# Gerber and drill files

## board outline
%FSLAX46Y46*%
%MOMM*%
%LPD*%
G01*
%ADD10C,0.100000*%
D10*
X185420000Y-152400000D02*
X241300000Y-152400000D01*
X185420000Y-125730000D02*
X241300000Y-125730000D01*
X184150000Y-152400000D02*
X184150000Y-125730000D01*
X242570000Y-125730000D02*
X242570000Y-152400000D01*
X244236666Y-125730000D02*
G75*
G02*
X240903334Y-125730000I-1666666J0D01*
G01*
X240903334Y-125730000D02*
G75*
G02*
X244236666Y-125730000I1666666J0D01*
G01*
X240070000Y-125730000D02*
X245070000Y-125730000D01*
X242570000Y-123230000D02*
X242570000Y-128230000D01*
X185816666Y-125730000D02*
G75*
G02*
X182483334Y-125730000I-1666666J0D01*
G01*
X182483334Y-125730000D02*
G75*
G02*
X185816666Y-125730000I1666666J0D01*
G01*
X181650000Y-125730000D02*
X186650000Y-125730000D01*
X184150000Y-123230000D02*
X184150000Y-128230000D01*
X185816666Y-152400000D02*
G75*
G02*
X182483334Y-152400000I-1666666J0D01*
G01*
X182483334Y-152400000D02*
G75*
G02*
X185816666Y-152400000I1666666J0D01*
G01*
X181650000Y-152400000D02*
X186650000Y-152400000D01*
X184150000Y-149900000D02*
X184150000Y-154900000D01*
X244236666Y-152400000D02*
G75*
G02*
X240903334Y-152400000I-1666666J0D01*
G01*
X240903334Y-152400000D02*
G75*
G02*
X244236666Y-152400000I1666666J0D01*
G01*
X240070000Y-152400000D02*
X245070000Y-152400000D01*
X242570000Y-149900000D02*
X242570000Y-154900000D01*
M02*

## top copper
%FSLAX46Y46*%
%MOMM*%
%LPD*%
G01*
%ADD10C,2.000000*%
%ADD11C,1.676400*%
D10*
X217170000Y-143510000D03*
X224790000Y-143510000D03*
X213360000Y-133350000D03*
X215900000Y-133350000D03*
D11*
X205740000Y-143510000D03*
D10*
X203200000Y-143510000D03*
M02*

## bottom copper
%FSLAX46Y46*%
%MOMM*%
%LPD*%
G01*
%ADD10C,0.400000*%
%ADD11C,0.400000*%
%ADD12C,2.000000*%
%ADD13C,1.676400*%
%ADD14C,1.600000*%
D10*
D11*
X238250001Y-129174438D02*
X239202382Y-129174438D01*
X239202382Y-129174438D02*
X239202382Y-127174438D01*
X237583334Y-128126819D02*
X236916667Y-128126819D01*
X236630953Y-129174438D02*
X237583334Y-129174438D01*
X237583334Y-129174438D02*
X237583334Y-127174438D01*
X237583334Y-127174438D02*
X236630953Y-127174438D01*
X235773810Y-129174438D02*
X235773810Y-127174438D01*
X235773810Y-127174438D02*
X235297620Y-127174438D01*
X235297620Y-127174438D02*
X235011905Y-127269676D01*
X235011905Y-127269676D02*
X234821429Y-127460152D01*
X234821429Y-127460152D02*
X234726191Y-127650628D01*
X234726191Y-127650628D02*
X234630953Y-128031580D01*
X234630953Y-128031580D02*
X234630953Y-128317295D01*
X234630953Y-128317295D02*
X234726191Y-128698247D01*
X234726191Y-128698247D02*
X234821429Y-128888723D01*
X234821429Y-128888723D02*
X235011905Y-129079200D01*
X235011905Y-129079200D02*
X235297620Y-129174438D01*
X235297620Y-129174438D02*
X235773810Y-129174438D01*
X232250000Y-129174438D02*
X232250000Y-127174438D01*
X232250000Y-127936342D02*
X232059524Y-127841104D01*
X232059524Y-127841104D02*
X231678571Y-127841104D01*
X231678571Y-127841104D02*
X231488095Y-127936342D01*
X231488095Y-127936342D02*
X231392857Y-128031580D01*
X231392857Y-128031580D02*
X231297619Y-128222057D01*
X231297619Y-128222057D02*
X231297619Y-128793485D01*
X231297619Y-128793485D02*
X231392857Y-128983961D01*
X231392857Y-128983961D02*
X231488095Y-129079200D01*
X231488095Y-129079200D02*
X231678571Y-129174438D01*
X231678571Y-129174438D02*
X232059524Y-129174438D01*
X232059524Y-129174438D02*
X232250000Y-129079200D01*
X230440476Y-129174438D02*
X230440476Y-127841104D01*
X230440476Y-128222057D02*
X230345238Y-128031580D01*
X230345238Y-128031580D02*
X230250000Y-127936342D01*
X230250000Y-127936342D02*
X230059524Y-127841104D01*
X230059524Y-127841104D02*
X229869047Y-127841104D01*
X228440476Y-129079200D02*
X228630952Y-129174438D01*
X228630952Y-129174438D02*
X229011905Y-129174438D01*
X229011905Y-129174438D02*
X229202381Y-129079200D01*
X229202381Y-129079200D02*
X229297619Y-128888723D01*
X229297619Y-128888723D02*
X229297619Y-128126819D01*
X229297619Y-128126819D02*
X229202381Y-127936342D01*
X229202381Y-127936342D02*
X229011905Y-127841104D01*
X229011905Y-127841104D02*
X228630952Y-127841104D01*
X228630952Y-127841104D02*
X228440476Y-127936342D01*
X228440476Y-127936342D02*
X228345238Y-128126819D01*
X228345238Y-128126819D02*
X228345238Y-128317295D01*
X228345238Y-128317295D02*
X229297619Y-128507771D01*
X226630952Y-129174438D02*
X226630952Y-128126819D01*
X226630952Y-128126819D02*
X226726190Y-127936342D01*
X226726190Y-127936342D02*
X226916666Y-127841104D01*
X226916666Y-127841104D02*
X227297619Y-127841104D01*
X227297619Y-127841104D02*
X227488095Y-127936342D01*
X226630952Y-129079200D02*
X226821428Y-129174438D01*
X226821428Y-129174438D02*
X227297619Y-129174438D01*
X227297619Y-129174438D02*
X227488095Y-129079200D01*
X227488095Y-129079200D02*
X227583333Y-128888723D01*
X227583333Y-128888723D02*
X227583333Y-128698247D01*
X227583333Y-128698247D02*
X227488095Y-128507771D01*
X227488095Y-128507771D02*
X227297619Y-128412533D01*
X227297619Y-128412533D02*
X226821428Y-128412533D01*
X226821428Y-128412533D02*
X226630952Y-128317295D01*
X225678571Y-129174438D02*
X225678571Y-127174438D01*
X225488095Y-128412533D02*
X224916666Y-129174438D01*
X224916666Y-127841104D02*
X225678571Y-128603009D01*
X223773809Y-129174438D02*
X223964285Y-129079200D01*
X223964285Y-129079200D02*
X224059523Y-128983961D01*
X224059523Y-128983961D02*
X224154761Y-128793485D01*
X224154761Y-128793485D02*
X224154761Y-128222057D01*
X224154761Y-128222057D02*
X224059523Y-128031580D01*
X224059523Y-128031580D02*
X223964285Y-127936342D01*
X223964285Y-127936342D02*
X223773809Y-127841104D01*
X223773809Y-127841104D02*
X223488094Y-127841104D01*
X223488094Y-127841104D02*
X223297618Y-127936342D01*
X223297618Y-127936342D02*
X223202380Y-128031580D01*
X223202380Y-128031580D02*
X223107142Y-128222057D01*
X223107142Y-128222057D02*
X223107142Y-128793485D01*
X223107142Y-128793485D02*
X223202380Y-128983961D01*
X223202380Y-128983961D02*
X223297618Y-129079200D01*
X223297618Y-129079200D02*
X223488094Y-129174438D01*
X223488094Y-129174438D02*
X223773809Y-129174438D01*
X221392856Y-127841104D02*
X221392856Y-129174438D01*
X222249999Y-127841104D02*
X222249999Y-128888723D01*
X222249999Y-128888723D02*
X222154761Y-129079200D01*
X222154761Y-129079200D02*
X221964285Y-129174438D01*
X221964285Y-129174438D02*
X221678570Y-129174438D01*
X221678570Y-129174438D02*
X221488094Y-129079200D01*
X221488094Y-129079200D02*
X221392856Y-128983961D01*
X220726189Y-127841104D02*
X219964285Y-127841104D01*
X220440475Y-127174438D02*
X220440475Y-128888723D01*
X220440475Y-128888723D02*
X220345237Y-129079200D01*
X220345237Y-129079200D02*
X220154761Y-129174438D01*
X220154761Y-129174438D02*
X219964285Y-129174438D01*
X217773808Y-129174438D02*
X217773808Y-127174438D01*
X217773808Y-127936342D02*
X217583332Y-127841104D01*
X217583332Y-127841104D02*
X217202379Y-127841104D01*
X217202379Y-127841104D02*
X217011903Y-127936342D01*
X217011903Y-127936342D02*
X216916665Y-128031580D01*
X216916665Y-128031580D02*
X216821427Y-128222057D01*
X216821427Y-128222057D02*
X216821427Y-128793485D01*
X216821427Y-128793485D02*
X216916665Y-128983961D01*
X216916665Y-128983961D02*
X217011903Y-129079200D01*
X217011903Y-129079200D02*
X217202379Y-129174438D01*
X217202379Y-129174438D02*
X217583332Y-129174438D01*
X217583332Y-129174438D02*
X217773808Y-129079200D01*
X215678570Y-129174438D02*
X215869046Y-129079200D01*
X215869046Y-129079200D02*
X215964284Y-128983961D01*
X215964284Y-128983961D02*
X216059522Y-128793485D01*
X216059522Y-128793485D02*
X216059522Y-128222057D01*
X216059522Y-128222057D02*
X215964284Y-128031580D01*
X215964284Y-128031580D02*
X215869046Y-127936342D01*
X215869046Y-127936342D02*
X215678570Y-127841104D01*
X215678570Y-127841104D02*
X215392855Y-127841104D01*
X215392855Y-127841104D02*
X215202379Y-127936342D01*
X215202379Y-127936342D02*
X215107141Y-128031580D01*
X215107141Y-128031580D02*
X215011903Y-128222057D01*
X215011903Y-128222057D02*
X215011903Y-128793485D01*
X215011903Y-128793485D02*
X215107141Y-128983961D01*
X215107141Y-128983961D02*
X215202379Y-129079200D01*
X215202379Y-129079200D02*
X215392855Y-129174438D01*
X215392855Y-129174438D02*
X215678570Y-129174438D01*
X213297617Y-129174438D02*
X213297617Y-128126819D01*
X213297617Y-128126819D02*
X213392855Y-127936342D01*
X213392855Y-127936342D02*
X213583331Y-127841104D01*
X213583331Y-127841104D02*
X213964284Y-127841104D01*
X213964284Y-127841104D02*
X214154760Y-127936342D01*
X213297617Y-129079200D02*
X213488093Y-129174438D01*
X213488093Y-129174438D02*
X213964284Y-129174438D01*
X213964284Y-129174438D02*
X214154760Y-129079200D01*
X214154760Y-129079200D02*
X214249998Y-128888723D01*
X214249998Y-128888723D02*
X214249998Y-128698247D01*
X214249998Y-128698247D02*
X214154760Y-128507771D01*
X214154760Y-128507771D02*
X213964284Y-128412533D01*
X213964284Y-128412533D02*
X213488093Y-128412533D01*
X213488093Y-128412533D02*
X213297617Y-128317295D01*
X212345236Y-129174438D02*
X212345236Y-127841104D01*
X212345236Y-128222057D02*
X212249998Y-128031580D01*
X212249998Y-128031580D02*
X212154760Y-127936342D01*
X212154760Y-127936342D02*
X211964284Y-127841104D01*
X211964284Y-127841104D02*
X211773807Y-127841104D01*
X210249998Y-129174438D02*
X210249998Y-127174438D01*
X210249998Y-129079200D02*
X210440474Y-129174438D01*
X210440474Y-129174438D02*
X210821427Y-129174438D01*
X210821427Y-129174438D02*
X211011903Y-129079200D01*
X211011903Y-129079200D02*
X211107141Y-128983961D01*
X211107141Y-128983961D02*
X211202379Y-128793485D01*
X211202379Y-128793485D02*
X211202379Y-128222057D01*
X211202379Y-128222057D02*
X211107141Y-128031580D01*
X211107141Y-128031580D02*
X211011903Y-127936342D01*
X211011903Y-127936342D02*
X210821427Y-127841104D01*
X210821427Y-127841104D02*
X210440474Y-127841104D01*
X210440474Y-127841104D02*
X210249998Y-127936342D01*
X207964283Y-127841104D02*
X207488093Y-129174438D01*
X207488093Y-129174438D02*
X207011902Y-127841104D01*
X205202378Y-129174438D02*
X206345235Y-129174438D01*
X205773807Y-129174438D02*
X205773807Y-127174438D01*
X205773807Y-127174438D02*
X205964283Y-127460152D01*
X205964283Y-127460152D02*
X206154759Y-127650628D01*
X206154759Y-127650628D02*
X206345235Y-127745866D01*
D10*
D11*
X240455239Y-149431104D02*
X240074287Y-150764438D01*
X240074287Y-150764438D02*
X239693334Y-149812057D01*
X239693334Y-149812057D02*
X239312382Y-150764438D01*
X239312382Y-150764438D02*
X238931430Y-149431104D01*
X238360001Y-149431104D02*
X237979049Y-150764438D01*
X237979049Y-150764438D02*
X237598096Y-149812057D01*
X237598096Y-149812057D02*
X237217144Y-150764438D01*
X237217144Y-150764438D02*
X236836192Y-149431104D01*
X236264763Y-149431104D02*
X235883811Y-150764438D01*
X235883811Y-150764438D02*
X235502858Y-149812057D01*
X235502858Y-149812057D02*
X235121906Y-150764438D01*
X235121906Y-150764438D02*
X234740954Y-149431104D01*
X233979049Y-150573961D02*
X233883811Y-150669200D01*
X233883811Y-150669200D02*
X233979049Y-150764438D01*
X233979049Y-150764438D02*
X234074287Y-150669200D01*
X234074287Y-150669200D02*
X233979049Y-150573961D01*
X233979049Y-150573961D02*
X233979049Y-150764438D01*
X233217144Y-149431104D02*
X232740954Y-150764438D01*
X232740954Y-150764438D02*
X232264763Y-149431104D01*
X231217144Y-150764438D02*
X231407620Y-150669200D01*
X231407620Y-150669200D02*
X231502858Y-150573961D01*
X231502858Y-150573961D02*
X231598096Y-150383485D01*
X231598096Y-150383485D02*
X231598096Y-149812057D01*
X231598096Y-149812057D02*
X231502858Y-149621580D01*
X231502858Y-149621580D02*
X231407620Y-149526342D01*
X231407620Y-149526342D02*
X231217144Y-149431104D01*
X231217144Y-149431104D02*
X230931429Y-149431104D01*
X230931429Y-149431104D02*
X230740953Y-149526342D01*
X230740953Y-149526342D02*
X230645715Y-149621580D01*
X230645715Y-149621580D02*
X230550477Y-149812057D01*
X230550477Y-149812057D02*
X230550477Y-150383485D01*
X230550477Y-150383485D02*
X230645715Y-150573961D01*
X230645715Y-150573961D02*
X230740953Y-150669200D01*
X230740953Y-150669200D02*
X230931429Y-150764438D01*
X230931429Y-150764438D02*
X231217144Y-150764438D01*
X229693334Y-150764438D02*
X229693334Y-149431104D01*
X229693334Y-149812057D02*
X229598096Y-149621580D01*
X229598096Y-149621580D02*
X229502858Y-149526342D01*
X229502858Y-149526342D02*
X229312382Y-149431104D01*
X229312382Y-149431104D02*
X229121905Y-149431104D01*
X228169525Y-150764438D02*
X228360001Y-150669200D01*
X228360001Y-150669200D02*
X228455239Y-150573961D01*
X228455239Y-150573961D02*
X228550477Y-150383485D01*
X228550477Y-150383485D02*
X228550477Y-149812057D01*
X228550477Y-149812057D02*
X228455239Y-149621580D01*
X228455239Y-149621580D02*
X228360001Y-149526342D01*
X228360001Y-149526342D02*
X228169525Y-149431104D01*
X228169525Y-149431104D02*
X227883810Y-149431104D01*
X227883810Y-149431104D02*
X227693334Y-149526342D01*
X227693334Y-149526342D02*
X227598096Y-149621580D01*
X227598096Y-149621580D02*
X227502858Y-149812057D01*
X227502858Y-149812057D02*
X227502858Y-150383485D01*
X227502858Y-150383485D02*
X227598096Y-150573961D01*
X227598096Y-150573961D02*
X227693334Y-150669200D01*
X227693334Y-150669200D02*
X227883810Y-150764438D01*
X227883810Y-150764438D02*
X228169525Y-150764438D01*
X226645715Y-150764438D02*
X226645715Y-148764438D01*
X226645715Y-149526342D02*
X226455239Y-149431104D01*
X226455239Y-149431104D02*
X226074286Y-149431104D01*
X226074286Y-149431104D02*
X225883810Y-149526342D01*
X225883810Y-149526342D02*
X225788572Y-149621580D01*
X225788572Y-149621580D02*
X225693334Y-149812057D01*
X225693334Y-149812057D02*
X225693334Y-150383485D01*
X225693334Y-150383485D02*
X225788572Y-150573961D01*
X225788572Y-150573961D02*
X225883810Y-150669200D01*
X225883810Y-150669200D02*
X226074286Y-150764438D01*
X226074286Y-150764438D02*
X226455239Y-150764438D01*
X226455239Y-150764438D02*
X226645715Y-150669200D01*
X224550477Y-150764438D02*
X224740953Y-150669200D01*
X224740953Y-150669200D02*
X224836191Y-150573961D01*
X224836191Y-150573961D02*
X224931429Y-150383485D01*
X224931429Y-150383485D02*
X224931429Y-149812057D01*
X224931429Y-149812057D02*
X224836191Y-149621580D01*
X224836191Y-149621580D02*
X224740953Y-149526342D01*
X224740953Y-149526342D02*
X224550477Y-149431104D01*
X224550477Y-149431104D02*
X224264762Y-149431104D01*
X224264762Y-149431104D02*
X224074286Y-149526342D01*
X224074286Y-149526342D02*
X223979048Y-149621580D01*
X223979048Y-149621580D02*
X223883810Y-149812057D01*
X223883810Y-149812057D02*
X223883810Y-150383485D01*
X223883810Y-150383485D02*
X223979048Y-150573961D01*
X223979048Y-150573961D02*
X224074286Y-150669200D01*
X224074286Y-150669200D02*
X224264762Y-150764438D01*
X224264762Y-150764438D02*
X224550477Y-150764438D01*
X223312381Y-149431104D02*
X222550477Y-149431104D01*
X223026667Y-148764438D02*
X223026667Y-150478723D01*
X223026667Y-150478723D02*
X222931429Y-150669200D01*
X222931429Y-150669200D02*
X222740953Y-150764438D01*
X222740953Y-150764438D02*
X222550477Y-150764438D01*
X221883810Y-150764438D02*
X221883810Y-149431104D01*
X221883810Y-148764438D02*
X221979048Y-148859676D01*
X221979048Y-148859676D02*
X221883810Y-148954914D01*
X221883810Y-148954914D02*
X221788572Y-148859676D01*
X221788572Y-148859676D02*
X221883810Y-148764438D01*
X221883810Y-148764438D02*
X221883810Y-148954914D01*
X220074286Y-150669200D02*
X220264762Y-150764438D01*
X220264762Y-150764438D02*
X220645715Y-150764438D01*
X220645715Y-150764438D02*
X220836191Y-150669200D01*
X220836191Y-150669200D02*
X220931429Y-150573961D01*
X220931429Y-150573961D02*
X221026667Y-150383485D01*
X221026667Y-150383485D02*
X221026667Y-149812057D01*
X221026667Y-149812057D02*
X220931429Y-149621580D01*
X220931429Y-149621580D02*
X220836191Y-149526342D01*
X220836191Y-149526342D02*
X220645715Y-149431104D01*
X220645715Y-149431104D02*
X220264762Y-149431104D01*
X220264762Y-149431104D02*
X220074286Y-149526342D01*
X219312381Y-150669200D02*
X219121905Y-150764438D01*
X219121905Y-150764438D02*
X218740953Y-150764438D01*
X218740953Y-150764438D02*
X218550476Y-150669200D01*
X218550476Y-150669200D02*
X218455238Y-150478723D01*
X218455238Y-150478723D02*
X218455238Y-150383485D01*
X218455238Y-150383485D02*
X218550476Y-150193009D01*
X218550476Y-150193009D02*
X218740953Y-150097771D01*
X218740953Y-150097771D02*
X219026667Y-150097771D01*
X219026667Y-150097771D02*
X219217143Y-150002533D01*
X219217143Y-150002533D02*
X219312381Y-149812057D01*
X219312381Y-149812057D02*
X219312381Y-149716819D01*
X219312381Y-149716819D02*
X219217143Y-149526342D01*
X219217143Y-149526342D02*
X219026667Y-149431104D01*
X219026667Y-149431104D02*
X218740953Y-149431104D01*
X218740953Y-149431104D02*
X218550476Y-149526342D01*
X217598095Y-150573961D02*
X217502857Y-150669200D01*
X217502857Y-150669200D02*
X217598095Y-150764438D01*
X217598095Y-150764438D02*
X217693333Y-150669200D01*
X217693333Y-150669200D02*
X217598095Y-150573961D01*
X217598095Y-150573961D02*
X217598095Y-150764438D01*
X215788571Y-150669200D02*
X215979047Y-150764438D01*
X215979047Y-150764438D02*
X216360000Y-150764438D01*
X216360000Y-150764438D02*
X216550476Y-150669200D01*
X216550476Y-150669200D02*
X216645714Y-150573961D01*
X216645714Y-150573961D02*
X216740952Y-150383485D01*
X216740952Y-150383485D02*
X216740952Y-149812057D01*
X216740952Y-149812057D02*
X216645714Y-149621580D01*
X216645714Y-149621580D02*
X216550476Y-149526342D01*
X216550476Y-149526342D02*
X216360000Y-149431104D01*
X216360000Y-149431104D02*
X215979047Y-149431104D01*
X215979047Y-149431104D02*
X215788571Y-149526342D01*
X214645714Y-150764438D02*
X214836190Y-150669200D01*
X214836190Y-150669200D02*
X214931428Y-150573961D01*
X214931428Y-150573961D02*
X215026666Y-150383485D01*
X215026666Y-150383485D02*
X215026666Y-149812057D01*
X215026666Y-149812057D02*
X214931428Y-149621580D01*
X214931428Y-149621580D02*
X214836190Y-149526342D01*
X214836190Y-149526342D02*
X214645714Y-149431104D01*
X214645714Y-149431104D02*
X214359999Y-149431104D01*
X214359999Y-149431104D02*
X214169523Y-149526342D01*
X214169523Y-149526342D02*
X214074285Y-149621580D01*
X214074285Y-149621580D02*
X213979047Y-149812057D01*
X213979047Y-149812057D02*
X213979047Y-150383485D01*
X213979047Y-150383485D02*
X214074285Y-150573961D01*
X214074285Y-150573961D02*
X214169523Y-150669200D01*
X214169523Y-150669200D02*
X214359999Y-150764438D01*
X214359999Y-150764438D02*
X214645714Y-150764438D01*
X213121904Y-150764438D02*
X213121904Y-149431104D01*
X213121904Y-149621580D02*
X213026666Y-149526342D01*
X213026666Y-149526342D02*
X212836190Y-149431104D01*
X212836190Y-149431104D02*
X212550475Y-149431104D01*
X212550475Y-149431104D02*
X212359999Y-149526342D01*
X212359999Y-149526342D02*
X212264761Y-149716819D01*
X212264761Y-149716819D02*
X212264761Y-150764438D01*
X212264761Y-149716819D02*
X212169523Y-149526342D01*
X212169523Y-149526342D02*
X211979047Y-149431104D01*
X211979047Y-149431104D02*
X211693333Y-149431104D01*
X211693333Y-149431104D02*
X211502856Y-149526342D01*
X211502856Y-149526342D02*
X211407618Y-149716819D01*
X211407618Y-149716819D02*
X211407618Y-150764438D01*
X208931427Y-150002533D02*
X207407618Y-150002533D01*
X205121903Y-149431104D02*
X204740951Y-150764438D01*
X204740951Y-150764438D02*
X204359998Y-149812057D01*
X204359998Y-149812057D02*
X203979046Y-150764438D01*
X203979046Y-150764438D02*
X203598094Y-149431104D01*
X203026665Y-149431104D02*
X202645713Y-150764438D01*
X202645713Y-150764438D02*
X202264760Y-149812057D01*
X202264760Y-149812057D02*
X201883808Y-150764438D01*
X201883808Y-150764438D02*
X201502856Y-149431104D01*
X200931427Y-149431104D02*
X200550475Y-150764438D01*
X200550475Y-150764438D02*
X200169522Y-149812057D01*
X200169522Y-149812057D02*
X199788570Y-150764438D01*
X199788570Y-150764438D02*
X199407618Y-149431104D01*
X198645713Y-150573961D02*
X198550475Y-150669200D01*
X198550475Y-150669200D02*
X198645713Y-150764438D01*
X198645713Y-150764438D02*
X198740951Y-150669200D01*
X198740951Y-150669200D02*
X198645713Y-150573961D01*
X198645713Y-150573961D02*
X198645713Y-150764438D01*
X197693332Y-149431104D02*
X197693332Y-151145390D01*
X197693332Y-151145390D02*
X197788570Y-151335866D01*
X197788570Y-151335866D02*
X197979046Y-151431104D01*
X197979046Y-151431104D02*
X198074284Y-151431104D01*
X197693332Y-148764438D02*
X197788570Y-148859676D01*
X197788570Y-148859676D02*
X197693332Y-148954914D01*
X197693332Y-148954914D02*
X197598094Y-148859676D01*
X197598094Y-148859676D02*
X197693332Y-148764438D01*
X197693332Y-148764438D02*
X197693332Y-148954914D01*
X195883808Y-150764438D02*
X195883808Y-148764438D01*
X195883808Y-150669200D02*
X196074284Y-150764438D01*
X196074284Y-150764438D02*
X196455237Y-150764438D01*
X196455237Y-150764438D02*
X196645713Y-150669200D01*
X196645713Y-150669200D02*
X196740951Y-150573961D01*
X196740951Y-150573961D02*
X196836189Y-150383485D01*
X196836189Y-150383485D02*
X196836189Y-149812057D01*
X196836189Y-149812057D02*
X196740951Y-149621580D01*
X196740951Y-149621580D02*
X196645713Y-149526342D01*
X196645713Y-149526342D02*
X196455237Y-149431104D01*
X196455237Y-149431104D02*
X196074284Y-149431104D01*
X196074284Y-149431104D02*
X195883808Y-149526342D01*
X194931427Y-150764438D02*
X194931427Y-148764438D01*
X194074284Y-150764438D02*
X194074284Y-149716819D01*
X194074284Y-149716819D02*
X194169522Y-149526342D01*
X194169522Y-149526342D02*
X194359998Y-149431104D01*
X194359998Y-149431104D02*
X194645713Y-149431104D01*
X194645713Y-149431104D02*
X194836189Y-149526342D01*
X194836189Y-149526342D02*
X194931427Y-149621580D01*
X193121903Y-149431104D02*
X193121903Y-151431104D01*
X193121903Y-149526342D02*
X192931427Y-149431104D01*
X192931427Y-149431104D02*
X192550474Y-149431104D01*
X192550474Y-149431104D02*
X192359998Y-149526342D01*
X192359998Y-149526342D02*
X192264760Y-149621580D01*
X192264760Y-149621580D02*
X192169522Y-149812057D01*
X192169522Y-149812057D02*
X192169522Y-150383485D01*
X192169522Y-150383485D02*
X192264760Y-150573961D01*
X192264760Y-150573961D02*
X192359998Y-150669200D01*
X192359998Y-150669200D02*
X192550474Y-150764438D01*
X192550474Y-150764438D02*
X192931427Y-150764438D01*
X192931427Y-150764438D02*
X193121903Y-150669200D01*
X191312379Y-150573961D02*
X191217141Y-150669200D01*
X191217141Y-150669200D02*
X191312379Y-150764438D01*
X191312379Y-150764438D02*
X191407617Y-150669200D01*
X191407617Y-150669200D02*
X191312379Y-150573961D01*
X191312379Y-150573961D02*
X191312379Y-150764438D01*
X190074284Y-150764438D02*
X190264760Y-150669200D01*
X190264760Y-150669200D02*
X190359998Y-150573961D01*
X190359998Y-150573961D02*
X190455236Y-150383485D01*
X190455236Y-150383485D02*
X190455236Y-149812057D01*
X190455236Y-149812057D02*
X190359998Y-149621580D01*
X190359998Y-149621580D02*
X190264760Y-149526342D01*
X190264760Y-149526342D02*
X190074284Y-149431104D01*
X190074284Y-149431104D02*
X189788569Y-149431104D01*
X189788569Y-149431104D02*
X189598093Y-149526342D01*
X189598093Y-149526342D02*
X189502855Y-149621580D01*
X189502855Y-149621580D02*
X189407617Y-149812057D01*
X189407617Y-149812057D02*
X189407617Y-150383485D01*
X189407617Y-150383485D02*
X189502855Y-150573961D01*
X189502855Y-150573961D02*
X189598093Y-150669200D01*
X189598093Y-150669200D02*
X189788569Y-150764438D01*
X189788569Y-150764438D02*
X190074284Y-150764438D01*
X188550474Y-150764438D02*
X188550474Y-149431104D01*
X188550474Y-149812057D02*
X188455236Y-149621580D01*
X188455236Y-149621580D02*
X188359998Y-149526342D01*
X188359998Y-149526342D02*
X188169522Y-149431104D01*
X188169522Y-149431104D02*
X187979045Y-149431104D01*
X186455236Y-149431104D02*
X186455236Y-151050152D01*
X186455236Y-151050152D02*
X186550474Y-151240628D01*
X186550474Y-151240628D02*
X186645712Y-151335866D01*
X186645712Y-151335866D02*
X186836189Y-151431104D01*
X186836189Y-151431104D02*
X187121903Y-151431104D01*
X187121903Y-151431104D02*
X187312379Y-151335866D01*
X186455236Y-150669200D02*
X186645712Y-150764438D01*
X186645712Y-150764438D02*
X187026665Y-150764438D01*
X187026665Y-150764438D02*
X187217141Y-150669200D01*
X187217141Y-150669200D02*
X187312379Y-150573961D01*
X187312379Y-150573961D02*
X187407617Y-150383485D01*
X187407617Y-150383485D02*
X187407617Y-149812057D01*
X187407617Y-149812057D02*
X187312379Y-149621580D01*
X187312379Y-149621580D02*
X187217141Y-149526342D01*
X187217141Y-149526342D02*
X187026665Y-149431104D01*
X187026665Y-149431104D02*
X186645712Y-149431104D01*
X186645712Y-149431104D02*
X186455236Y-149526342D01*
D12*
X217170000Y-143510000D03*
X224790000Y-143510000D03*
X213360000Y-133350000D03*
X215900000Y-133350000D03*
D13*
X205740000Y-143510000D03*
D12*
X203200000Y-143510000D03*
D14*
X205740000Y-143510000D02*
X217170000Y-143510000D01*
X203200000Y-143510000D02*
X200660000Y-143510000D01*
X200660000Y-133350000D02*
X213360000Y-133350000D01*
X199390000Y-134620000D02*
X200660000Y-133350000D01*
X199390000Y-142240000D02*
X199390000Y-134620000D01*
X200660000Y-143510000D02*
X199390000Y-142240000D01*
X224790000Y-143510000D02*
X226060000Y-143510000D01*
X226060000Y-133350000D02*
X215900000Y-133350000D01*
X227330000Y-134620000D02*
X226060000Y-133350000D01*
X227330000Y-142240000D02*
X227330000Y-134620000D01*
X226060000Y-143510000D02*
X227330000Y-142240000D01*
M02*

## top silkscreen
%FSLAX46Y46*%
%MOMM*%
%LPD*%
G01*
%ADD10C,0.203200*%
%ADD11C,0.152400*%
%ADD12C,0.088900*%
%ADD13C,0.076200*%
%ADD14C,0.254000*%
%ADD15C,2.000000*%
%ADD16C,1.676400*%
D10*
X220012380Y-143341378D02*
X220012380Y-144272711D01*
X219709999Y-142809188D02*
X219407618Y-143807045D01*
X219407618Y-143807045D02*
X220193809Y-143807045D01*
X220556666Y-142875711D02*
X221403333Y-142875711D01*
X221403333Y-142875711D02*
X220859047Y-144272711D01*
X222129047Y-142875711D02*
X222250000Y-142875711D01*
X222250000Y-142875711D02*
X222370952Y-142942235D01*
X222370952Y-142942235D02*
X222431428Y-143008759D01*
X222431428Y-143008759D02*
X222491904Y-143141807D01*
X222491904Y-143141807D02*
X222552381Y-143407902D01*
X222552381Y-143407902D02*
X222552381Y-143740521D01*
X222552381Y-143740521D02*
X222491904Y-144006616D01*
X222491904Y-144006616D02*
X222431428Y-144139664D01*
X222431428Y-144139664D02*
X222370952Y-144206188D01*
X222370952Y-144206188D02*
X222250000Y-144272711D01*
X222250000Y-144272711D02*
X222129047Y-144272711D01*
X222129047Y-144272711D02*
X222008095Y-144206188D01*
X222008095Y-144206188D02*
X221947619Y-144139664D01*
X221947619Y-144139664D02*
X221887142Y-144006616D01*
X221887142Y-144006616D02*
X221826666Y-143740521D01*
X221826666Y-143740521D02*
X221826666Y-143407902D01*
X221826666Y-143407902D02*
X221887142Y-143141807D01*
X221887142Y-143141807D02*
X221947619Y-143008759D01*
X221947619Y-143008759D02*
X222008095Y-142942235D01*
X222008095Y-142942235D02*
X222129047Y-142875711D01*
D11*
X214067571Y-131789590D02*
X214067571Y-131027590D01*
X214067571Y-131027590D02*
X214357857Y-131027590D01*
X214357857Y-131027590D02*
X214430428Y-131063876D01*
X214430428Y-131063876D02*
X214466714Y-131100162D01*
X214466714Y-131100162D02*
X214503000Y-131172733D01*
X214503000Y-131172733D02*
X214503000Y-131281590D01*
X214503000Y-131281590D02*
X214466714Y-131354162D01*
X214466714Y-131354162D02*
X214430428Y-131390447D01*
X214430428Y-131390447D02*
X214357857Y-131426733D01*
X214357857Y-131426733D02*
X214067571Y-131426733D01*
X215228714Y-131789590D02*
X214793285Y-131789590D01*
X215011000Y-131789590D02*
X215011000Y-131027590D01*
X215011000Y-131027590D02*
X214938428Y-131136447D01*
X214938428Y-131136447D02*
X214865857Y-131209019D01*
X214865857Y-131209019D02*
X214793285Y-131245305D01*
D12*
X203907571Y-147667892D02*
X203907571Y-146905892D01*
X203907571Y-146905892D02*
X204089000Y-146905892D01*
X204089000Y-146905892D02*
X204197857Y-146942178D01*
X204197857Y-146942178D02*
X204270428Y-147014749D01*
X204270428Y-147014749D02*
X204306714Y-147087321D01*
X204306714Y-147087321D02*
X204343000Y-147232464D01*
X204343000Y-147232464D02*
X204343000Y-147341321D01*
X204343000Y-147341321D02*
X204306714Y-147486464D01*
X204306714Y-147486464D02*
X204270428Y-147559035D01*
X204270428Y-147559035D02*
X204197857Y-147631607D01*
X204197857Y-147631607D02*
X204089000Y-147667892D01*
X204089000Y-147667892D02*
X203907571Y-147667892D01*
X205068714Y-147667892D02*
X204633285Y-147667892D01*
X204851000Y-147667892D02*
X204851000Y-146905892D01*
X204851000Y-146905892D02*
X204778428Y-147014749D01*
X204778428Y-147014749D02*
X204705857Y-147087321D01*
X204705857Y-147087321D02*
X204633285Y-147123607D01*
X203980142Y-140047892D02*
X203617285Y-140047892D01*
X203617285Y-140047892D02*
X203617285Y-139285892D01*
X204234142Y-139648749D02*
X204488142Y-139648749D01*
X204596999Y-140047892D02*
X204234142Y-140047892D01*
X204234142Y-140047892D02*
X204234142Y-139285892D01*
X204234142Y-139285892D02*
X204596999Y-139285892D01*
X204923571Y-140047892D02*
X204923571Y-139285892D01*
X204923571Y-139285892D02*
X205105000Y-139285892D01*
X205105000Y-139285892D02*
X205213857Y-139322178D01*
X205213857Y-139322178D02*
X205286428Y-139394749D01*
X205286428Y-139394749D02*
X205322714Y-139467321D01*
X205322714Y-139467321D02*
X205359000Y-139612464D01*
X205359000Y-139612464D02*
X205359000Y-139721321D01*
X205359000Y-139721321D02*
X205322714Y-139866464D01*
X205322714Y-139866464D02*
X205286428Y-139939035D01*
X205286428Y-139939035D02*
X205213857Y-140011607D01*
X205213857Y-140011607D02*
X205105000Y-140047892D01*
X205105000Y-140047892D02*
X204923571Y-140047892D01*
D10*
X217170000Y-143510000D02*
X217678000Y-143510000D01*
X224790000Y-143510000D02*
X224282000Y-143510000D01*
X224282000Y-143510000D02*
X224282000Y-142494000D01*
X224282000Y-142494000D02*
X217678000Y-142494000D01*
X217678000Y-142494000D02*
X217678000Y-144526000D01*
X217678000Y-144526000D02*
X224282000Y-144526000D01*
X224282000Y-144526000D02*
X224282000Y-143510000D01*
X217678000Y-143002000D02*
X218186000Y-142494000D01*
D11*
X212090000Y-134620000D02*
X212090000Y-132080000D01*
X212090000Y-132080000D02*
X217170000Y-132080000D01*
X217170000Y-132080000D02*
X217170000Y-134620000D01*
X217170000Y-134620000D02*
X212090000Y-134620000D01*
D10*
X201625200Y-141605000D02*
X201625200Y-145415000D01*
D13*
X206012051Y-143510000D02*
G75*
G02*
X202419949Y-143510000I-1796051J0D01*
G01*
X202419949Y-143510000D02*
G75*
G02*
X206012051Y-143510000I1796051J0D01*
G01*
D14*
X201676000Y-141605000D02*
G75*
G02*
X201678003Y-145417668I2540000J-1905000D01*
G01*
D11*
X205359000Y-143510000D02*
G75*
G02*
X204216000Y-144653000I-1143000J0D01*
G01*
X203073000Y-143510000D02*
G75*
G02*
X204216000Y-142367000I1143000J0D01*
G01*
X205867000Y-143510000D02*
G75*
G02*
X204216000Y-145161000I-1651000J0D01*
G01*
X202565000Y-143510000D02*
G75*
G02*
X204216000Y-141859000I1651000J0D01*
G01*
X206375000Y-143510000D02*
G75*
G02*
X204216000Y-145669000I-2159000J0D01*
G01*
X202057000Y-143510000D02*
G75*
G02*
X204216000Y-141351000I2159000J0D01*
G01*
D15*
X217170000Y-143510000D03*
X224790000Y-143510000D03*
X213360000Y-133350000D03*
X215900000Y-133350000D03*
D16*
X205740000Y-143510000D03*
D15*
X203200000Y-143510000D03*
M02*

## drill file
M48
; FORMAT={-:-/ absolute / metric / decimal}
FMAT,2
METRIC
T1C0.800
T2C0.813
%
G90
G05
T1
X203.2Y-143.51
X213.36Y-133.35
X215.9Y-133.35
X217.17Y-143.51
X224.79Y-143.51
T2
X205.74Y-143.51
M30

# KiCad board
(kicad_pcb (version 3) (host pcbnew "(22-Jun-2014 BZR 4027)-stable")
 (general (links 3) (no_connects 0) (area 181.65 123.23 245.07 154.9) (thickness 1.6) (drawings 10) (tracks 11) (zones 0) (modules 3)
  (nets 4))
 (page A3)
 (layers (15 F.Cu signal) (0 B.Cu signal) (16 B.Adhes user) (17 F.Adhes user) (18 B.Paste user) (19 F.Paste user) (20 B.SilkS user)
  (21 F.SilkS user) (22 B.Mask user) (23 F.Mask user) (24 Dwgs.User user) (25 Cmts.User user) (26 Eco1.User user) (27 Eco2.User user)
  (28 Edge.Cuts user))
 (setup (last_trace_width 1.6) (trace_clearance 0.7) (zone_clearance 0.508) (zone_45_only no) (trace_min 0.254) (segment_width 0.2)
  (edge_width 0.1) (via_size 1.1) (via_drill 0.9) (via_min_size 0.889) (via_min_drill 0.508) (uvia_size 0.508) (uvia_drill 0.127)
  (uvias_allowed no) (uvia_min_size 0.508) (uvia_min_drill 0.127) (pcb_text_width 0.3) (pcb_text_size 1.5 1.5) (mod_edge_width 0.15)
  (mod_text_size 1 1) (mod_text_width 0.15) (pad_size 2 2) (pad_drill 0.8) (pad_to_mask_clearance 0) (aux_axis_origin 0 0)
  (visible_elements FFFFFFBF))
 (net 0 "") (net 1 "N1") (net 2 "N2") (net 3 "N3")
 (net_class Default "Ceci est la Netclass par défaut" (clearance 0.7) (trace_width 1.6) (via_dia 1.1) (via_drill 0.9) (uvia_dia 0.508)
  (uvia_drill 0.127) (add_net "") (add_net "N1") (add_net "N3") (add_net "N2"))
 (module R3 (layer F.Cu) (at 220.98 143.51) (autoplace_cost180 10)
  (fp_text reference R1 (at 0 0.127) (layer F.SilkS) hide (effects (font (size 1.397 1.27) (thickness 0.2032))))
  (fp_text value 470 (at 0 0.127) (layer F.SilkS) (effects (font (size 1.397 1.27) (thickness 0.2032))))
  (fp_line (start -3.81 0) (end -3.302 0) (layer F.SilkS) (width 0.2032))
  (fp_line (start 3.81 0) (end 3.302 0) (layer F.SilkS) (width 0.2032))
  (fp_line (start 3.302 0) (end 3.302 -1.016) (layer F.SilkS) (width 0.2032))
  (fp_line (start 3.302 -1.016) (end -3.302 -1.016) (layer F.SilkS) (width 0.2032))
  (fp_line (start -3.302 -1.016) (end -3.302 1.016) (layer F.SilkS) (width 0.2032))
  (fp_line (start -3.302 1.016) (end 3.302 1.016) (layer F.SilkS) (width 0.2032))
  (fp_line (start 3.302 1.016) (end 3.302 0) (layer F.SilkS) (width 0.2032))
  (fp_line (start -3.302 -0.508) (end -2.794 -1.016) (layer F.SilkS) (width 0.2032))
  (pad 1 thru_hole circle (at -3.81 0) (size 2 2) (drill 0.8) (layers *.Cu *.Mask F.SilkS) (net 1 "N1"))
  (pad 2 thru_hole circle (at 3.81 0) (size 2 2) (drill 0.8) (layers *.Cu *.Mask F.SilkS) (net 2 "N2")))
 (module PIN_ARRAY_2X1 (layer F.Cu) (at 214.63 133.35)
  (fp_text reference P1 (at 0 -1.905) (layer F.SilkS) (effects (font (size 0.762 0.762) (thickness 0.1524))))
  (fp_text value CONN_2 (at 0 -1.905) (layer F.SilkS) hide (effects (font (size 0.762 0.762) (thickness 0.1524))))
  (fp_line (start -2.54 1.27) (end -2.54 -1.27) (layer F.SilkS) (width 0.1524))
  (fp_line (start -2.54 -1.27) (end 2.54 -1.27) (layer F.SilkS) (width 0.1524))
  (fp_line (start 2.54 -1.27) (end 2.54 1.27) (layer F.SilkS) (width 0.1524))
  (fp_line (start 2.54 1.27) (end -2.54 1.27) (layer F.SilkS) (width 0.1524))
  (pad 1 thru_hole circle (at -1.27 0) (size 2 2) (drill 0.8) (layers *.Cu *.Mask F.SilkS) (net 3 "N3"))
  (pad 2 thru_hole circle (at 1.27 0) (size 2 2) (drill 0.8) (layers *.Cu *.Mask F.SilkS) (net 2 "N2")))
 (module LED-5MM (layer F.Cu) (at 204.47 143.51 180)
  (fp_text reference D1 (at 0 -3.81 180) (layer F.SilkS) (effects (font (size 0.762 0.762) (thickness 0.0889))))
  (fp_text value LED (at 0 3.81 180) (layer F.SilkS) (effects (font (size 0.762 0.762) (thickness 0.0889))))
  (fp_line (start 2.8448 1.905) (end 2.8448 -1.905) (layer F.SilkS) (width 0.2032))
  (fp_circle (center 0.254 0) (end -1.016 1.27) (layer F.SilkS) (width 0.0762))
  (fp_arc (start 0.254 0) (end 2.794 1.905) (angle 286.2) (layer F.SilkS) (width 0.254))
  (fp_arc (start 0.254 0) (end -0.889 0) (angle 90) (layer F.SilkS) (width 0.1524))
  (fp_arc (start 0.254 0) (end 1.397 0) (angle 90) (layer F.SilkS) (width 0.1524))
  (fp_arc (start 0.254 0) (end -1.397 0) (angle 90) (layer F.SilkS) (width 0.1524))
  (fp_arc (start 0.254 0) (end 1.905 0) (angle 90) (layer F.SilkS) (width 0.1524))
  (fp_arc (start 0.254 0) (end -1.905 0) (angle 90) (layer F.SilkS) (width 0.1524))
  (fp_arc (start 0.254 0) (end 2.413 0) (angle 90) (layer F.SilkS) (width 0.1524))
  (pad 1 thru_hole circle (at -1.27 0 180) (size 1.6764 1.6764) (drill 0.8128) (layers *.Cu *.Mask F.SilkS) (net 1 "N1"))
  (pad 2 thru_hole circle (at 1.27 0 180) (size 2 2) (drill 0.8) (layers *.Cu *.Mask F.SilkS) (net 3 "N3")))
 (gr_line (start 185.42 152.4) (end 241.3 152.4) (angle 90) (layer Edge.Cuts) (width 0.1))
 (gr_line (start 185.42 125.73) (end 241.3 125.73) (angle 90) (layer Edge.Cuts) (width 0.1))
 (gr_line (start 184.15 152.4) (end 184.15 125.73) (angle 90) (layer Edge.Cuts) (width 0.1))
 (gr_line (start 242.57 125.73) (end 242.57 152.4) (angle 90) (layer Edge.Cuts) (width 0.1))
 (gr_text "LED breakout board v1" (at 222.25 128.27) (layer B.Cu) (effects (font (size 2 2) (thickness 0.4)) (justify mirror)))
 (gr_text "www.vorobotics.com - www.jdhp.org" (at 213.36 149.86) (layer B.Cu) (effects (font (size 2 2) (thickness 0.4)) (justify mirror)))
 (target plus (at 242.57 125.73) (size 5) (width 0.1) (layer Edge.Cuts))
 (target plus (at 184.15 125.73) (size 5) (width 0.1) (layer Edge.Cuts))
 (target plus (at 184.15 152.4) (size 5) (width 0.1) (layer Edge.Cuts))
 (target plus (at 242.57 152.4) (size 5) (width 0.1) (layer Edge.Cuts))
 (segment (start 205.74 143.51) (end 217.17 143.51) (width 1.6) (layer B.Cu) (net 1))
 (segment (start 203.2 143.51) (end 200.66 143.51) (width 1.6) (layer B.Cu) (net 3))
 (segment (start 200.66 133.35) (end 213.36 133.35) (width 1.6) (layer B.Cu) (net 3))
 (segment (start 199.39 134.62) (end 200.66 133.35) (width 1.6) (layer B.Cu) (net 3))
 (segment (start 199.39 142.24) (end 199.39 134.62) (width 1.6) (layer B.Cu) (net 3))
 (segment (start 200.66 143.51) (end 199.39 142.24) (width 1.6) (layer B.Cu) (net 3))
 (segment (start 224.79 143.51) (end 226.06 143.51) (width 1.6) (layer B.Cu) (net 2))
 (segment (start 226.06 133.35) (end 215.9 133.35) (width 1.6) (layer B.Cu) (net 2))
 (segment (start 227.33 134.62) (end 226.06 133.35) (width 1.6) (layer B.Cu) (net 2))
 (segment (start 227.33 142.24) (end 227.33 134.62) (width 1.6) (layer B.Cu) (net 2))
 (segment (start 226.06 143.51) (end 227.33 142.24) (width 1.6) (layer B.Cu) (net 2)))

